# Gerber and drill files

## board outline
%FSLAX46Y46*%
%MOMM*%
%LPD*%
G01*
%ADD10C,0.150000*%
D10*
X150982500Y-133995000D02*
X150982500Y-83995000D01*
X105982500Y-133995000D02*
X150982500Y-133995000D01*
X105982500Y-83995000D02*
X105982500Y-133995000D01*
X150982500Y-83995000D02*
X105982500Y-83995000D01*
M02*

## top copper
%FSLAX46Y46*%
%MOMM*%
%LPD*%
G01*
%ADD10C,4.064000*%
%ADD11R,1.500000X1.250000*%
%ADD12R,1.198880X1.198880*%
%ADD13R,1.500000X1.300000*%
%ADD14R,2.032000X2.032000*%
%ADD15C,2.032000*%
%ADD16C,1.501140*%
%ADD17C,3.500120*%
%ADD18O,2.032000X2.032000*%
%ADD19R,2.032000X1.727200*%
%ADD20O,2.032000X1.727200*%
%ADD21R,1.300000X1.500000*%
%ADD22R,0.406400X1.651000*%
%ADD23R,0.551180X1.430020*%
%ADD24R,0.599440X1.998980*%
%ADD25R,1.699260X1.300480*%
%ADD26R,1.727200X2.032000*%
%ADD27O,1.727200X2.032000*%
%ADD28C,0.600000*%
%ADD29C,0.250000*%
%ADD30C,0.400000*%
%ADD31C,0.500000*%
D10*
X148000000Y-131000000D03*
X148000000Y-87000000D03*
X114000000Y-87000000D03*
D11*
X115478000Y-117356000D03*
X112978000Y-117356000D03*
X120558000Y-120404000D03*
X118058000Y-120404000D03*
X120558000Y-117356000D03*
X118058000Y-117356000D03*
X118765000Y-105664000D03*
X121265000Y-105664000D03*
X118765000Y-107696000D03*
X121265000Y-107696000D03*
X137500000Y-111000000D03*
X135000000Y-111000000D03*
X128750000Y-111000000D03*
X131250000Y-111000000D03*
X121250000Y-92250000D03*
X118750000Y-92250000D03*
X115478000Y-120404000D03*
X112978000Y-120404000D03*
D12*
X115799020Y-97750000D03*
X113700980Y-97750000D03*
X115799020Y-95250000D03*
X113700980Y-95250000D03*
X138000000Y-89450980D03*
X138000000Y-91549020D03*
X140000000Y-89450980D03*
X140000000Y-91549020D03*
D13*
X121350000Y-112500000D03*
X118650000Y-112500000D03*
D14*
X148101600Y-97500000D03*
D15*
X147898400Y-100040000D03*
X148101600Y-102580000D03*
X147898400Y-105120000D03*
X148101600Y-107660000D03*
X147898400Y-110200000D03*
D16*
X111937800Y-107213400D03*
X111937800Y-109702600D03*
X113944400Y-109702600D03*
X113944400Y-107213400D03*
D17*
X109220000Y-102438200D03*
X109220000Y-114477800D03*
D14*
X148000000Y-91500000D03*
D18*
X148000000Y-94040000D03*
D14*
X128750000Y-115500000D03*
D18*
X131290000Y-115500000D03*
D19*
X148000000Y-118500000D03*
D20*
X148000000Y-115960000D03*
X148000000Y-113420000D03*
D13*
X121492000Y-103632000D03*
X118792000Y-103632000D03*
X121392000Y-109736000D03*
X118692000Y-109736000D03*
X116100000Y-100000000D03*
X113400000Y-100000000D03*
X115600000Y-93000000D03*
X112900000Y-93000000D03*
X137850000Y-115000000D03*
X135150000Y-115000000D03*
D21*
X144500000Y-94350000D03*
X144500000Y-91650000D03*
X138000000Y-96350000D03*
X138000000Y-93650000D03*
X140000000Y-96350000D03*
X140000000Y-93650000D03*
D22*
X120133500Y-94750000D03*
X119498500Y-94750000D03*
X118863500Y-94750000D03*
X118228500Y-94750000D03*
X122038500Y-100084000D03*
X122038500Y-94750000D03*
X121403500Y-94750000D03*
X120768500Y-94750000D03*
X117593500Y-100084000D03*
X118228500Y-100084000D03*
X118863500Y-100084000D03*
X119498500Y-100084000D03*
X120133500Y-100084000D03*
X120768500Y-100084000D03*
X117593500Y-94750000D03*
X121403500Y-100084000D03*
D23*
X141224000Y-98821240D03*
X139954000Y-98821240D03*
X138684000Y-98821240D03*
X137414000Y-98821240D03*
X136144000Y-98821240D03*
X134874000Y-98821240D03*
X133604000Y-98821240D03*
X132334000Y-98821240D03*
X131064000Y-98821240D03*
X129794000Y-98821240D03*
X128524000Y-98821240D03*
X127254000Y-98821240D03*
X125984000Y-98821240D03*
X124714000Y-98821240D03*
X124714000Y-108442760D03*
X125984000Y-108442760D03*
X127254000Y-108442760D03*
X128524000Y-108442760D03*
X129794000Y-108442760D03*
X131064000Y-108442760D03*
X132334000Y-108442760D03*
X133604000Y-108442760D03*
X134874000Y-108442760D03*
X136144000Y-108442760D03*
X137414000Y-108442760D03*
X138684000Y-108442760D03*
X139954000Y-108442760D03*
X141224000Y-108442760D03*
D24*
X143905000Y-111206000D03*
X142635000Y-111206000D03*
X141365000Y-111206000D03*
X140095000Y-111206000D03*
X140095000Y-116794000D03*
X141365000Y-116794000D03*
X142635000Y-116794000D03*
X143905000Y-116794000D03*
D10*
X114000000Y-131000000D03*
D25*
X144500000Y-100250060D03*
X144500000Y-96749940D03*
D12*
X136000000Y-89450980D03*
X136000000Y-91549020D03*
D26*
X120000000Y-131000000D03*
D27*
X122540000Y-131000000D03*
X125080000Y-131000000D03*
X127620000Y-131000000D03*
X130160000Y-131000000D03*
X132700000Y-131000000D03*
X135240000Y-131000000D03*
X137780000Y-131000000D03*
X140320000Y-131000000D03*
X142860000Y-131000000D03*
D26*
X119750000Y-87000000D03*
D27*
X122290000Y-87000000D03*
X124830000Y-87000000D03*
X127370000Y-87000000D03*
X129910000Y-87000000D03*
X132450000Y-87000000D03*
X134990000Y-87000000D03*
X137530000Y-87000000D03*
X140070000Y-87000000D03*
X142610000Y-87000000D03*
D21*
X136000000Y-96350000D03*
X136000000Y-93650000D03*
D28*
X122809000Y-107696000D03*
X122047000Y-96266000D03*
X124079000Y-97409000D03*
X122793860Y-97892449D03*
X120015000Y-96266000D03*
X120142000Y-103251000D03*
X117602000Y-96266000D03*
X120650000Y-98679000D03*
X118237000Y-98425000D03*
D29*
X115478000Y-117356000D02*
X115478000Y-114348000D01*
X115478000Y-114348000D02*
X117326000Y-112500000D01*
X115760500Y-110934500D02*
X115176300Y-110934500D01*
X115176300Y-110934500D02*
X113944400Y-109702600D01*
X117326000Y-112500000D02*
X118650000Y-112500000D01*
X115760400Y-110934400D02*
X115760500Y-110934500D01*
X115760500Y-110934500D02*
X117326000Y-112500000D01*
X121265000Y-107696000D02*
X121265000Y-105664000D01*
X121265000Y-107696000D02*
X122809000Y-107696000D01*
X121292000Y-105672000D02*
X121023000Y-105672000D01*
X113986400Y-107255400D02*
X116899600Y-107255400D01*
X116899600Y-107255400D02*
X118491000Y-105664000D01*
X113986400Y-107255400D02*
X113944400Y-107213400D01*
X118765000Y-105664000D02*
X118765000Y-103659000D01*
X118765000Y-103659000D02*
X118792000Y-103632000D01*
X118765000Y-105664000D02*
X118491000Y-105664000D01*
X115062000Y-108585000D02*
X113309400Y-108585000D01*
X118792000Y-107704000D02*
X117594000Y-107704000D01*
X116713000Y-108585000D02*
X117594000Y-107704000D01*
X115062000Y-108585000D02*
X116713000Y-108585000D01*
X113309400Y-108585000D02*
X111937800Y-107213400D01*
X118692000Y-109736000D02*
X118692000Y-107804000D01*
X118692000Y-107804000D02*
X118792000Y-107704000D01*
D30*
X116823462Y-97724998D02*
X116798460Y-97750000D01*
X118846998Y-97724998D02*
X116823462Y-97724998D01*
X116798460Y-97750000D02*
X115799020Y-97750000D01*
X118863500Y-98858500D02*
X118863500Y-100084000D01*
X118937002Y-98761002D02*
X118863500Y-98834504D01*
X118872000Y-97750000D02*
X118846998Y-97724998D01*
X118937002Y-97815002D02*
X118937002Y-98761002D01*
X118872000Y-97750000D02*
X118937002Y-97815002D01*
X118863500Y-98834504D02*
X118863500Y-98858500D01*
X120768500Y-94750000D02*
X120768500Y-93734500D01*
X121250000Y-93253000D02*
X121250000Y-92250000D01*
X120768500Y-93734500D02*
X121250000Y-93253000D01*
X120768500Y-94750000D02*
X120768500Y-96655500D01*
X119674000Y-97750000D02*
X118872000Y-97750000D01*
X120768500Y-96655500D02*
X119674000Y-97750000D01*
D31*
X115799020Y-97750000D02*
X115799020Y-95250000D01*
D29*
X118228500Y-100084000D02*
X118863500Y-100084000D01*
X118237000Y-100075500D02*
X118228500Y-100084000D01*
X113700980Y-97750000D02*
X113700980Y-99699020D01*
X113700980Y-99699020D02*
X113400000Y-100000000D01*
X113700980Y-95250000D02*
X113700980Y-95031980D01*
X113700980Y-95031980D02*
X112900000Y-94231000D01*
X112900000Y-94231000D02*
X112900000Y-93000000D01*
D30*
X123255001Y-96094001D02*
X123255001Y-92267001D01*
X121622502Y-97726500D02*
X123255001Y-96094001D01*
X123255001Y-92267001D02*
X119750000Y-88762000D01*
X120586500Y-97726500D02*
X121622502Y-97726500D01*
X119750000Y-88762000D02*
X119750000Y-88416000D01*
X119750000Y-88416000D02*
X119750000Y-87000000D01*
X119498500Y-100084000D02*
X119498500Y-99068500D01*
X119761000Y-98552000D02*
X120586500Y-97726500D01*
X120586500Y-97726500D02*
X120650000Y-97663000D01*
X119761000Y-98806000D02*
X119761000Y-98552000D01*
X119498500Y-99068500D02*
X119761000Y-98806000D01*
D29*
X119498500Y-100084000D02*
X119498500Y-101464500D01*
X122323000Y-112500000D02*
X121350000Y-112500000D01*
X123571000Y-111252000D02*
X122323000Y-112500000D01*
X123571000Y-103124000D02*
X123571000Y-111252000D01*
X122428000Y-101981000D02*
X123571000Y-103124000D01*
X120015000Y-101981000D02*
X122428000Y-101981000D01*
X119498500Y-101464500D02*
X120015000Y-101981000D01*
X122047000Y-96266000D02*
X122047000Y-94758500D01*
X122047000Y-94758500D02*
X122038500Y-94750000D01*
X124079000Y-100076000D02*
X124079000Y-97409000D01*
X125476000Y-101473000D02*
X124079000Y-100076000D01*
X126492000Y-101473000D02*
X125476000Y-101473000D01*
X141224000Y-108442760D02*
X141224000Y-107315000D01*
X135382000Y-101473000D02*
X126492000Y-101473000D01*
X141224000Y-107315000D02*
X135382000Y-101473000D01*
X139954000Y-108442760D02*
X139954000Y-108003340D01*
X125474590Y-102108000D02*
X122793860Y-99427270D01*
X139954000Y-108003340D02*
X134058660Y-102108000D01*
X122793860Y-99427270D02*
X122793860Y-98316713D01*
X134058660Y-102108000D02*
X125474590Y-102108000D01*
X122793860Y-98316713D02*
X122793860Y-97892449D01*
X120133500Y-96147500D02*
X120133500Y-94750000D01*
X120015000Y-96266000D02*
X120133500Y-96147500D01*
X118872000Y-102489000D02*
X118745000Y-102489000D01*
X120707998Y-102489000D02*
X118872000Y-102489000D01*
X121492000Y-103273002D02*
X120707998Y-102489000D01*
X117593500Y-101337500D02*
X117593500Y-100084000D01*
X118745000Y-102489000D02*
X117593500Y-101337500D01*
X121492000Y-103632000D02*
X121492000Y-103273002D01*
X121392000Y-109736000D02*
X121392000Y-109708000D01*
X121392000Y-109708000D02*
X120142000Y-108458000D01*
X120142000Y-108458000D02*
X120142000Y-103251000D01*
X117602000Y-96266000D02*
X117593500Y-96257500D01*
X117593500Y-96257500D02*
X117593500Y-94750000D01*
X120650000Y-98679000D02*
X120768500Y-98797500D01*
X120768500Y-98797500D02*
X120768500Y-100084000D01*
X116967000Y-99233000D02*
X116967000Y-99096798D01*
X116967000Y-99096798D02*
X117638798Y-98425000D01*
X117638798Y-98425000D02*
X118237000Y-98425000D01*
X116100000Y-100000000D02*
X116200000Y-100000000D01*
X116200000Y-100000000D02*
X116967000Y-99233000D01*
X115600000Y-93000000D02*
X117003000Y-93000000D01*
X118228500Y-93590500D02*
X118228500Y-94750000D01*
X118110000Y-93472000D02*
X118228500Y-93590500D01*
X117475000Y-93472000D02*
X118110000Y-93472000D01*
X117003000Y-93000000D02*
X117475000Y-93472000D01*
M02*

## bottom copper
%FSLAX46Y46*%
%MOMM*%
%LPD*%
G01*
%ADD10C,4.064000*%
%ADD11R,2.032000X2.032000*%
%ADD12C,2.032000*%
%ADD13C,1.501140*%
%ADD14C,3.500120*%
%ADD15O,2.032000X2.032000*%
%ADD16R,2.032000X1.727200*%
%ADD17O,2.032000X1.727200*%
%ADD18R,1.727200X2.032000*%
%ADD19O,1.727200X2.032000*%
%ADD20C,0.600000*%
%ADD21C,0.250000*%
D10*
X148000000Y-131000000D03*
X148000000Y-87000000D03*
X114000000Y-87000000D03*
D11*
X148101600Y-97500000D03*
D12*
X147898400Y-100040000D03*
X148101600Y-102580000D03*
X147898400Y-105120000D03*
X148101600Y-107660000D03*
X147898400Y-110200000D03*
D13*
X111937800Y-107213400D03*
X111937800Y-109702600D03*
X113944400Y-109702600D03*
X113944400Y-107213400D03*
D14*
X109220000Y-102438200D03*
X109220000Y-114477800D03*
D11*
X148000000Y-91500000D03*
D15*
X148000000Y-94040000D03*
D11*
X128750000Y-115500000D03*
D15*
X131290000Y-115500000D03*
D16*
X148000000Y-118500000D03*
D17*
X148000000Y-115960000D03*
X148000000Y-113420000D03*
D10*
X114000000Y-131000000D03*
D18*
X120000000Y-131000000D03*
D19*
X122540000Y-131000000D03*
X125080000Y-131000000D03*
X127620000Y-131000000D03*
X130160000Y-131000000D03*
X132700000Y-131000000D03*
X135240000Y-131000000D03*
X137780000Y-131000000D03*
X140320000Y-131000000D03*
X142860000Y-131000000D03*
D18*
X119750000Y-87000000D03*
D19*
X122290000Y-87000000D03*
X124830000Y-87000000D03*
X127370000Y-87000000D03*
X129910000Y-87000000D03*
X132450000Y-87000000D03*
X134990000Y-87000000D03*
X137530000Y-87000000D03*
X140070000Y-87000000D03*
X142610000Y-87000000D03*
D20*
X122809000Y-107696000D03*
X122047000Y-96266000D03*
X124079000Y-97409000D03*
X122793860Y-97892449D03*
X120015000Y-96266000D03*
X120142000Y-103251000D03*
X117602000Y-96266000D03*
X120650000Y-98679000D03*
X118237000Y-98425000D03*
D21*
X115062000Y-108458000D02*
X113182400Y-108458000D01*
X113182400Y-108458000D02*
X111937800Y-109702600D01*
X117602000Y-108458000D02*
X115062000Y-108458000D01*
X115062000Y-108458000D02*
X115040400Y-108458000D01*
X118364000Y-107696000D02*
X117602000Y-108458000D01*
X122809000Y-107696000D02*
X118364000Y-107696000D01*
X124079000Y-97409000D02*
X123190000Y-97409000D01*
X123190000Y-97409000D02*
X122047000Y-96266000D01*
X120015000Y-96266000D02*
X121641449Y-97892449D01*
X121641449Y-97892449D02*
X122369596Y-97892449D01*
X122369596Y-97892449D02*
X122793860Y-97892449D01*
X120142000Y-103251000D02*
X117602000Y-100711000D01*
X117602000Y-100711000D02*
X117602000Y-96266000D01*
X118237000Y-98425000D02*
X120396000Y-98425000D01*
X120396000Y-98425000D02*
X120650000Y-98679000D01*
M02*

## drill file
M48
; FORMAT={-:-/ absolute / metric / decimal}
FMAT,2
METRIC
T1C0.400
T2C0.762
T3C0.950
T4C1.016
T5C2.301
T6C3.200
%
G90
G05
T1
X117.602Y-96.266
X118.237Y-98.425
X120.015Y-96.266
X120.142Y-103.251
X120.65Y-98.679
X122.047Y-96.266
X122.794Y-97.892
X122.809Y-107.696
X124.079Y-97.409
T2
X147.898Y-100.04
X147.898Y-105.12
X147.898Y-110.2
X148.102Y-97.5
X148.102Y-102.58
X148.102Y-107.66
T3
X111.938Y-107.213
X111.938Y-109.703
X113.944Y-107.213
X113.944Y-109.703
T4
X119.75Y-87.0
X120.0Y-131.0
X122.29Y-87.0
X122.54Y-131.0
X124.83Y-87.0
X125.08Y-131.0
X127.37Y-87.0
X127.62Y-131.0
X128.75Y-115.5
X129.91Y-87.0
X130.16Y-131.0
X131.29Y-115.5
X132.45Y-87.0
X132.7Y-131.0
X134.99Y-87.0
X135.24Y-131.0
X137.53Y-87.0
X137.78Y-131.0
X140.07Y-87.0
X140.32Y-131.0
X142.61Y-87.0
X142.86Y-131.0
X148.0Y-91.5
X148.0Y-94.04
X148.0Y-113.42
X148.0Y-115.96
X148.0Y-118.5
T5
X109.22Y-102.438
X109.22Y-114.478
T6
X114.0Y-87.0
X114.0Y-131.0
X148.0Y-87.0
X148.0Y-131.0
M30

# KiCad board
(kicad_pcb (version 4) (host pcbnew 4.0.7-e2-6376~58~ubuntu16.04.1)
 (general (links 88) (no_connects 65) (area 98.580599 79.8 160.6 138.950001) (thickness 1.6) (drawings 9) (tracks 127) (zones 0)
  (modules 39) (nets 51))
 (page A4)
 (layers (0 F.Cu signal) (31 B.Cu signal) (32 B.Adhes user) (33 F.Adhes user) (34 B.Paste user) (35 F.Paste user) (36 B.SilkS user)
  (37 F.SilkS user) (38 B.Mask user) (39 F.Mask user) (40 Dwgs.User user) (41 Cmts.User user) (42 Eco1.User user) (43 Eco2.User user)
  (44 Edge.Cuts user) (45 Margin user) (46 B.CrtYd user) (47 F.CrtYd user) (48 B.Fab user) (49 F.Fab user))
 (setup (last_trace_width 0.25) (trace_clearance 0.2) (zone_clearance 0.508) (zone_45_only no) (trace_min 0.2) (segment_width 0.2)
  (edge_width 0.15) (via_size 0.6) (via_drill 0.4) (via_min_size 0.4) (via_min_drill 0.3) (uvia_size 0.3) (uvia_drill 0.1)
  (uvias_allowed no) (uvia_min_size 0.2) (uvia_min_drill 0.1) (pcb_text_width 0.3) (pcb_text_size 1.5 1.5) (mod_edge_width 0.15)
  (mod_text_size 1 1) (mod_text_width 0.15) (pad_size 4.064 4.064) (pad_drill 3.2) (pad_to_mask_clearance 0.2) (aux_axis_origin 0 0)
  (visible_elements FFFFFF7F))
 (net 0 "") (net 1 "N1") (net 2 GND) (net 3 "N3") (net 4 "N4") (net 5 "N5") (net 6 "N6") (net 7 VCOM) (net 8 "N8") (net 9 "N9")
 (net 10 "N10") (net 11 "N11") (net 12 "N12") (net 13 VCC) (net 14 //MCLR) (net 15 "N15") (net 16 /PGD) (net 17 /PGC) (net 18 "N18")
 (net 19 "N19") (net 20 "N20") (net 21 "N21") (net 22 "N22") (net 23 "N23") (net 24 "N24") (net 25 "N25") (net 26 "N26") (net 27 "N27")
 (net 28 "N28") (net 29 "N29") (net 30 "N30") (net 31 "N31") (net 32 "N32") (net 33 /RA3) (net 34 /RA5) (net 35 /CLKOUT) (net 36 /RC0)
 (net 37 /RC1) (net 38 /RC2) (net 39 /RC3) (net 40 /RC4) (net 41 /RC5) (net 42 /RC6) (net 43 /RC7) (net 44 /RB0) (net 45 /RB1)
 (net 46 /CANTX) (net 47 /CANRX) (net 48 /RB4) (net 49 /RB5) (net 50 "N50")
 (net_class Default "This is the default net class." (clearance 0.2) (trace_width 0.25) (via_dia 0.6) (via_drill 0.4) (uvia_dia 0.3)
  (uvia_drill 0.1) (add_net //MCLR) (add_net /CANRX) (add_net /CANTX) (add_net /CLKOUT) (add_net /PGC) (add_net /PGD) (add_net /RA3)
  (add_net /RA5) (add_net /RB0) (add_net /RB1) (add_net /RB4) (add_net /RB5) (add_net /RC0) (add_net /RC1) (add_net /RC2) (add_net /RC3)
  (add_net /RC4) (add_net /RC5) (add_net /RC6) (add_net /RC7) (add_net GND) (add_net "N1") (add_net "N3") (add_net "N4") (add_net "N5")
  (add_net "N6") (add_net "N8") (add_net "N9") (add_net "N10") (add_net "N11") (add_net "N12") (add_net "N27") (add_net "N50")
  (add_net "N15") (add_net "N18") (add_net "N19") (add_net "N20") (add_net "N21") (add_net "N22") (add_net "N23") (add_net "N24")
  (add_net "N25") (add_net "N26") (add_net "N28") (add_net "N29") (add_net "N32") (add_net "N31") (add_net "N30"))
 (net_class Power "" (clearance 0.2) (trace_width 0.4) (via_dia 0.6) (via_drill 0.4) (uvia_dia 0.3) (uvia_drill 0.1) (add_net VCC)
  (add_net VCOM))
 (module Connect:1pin (layer F.Cu) (at 148 131 180)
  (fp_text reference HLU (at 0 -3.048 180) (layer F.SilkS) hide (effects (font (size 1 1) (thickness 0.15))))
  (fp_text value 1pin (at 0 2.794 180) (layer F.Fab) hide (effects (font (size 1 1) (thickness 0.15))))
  (pad 1 thru_hole circle (at 0 0 180) (size 4.064 4.064) (drill 3.2) (layers *.Cu *.Mask F.SilkS)))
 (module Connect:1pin (layer F.Cu) (at 148 87 180)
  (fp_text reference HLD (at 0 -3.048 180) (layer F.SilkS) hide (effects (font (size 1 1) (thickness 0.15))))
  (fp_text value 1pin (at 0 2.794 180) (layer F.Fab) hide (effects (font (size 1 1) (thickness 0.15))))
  (pad 1 thru_hole circle (at 0 0 180) (size 4.064 4.064) (drill 3.2) (layers *.Cu *.Mask F.SilkS)))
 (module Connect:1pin (layer F.Cu) (at 114 87 180)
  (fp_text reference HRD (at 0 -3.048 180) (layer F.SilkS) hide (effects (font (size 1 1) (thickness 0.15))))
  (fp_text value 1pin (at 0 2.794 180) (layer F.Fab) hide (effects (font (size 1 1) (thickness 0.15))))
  (pad 1 thru_hole circle (at 0 0 180) (size 4.064 4.064) (drill 3.2) (layers *.Cu *.Mask F.SilkS)))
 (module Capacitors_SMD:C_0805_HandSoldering (layer F.Cu) (at 114.228 117.356 180)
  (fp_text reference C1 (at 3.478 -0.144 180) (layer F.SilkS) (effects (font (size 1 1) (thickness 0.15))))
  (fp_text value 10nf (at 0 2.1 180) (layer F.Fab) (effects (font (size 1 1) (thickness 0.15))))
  (pad 1 smd rect (at -1.25 0 180) (size 1.5 1.25) (layers F.Cu F.Paste F.Mask) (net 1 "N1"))
  (pad 2 smd rect (at 1.25 0 180) (size 1.5 1.25) (layers F.Cu F.Paste F.Mask) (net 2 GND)))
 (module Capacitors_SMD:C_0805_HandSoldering (layer F.Cu) (at 119.308 120.404 180)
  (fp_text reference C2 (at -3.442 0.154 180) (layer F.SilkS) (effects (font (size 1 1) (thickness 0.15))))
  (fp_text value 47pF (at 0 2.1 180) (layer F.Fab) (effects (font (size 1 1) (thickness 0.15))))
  (pad 1 smd rect (at -1.25 0 180) (size 1.5 1.25) (layers F.Cu F.Paste F.Mask) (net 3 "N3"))
  (pad 2 smd rect (at 1.25 0 180) (size 1.5 1.25) (layers F.Cu F.Paste F.Mask) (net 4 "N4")))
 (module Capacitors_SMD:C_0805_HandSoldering (layer F.Cu) (at 119.308 117.356 180)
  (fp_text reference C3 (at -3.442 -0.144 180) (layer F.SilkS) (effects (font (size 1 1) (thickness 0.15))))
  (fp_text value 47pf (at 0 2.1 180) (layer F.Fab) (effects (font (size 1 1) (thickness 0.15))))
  (pad 1 smd rect (at -1.25 0 180) (size 1.5 1.25) (layers F.Cu F.Paste F.Mask) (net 3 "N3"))
  (pad 2 smd rect (at 1.25 0 180) (size 1.5 1.25) (layers F.Cu F.Paste F.Mask) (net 4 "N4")))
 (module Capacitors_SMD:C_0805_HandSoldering (layer F.Cu) (at 120.015 105.664)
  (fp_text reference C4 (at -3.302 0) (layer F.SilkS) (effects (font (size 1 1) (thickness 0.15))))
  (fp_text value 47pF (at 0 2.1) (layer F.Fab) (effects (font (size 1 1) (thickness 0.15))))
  (pad 1 smd rect (at -1.25 0) (size 1.5 1.25) (layers F.Cu F.Paste F.Mask) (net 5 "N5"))
  (pad 2 smd rect (at 1.25 0) (size 1.5 1.25) (layers F.Cu F.Paste F.Mask) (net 2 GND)))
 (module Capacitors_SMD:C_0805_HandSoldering (layer F.Cu) (at 120.015 107.696)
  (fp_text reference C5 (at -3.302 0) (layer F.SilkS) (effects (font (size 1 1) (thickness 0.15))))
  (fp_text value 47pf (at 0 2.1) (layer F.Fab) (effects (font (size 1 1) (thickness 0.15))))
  (pad 1 smd rect (at -1.25 0) (size 1.5 1.25) (layers F.Cu F.Paste F.Mask) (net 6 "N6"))
  (pad 2 smd rect (at 1.25 0) (size 1.5 1.25) (layers F.Cu F.Paste F.Mask) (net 2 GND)))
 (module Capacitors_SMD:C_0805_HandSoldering (layer F.Cu) (at 136.25 111 180)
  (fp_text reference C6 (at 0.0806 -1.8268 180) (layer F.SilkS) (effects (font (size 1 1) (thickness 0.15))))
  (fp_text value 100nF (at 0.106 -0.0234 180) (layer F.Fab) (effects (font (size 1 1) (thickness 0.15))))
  (pad 1 smd rect (at -1.25 0 180) (size 1.5 1.25) (layers F.Cu F.Paste F.Mask) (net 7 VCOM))
  (pad 2 smd rect (at 1.25 0 180) (size 1.5 1.25) (layers F.Cu F.Paste F.Mask) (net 2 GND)))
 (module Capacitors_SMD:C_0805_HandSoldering (layer F.Cu) (at 130 111)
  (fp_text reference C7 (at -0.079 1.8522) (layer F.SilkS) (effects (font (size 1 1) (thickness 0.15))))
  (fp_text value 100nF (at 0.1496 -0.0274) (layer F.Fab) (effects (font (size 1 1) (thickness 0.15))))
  (pad 1 smd rect (at -1.25 0) (size 1.5 1.25) (layers F.Cu F.Paste F.Mask) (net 7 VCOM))
  (pad 2 smd rect (at 1.25 0) (size 1.5 1.25) (layers F.Cu F.Paste F.Mask) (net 2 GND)))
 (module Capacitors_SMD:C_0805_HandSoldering (layer F.Cu) (at 120 92.25 180)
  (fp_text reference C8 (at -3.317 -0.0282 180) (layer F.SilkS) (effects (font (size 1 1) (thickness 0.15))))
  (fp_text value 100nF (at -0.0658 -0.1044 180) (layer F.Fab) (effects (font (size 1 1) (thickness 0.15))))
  (pad 1 smd rect (at -1.25 0 180) (size 1.5 1.25) (layers F.Cu F.Paste F.Mask) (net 7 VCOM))
  (pad 2 smd rect (at 1.25 0 180) (size 1.5 1.25) (layers F.Cu F.Paste F.Mask) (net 2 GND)))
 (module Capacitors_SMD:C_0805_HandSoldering (layer F.Cu) (at 114.228 120.404 180)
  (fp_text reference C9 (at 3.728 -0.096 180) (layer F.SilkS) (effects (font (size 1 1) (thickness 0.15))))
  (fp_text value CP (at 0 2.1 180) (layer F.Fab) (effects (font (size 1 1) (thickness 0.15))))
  (pad 1 smd rect (at -1.25 0 180) (size 1.5 1.25) (layers F.Cu F.Paste F.Mask) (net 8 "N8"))
  (pad 2 smd rect (at 1.25 0 180) (size 1.5 1.25) (layers F.Cu F.Paste F.Mask) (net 2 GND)))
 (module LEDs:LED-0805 (layer F.Cu) (at 114.75 97.75)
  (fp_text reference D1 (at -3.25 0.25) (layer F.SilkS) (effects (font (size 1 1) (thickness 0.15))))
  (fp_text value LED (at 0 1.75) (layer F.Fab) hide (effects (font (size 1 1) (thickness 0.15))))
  (pad 2 smd rect (at 1.04902 0 180) (size 1.19888 1.19888) (layers F.Cu F.Paste F.Mask) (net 7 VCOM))
  (pad 1 smd rect (at -1.04902 0 180) (size 1.19888 1.19888) (layers F.Cu F.Paste F.Mask) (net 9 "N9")))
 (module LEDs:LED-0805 (layer F.Cu) (at 114.75 95.25)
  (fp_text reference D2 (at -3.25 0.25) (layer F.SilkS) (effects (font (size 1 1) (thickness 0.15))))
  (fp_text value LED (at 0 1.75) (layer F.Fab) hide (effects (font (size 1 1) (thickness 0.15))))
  (pad 2 smd rect (at 1.04902 0 180) (size 1.19888 1.19888) (layers F.Cu F.Paste F.Mask) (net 7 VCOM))
  (pad 1 smd rect (at -1.04902 0 180) (size 1.19888 1.19888) (layers F.Cu F.Paste F.Mask) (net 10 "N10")))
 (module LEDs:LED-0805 (layer F.Cu) (at 138 90.5 90)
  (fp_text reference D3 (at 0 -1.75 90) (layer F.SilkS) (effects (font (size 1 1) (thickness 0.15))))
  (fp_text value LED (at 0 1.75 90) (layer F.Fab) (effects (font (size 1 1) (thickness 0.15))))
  (pad 2 smd rect (at 1.04902 0 270) (size 1.19888 1.19888) (layers F.Cu F.Paste F.Mask) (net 7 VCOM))
  (pad 1 smd rect (at -1.04902 0 270) (size 1.19888 1.19888) (layers F.Cu F.Paste F.Mask) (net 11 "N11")))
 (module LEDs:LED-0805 (layer F.Cu) (at 140 90.5 90)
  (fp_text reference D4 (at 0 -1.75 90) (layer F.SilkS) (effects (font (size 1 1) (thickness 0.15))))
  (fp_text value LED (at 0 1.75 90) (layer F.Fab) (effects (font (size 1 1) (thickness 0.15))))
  (pad 2 smd rect (at 1.04902 0 270) (size 1.19888 1.19888) (layers F.Cu F.Paste F.Mask) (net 7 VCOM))
  (pad 1 smd rect (at -1.04902 0 270) (size 1.19888 1.19888) (layers F.Cu F.Paste F.Mask) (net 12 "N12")))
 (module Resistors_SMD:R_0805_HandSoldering (layer F.Cu) (at 120 112.5 180)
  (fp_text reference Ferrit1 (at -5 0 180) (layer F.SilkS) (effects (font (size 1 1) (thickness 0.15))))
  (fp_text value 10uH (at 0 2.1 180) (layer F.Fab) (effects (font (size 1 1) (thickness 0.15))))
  (pad 1 smd rect (at -1.35 0 180) (size 1.5 1.3) (layers F.Cu F.Paste F.Mask) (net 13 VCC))
  (pad 2 smd rect (at 1.35 0 180) (size 1.5 1.3) (layers F.Cu F.Paste F.Mask) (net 1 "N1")))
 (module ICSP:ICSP (layer F.Cu) (at 148 97.5 270)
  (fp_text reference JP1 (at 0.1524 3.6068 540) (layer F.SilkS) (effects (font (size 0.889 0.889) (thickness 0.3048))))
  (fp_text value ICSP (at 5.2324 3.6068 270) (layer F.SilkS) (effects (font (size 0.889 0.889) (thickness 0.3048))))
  (pad 1 thru_hole rect (at 0 -0.1016 270) (size 2.032 2.032) (drill 0.762) (layers *.Cu *.Mask F.SilkS) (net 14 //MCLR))
  (pad 2 thru_hole circle (at 2.54 0.1016 270) (size 2.032 2.032) (drill 0.762) (layers *.Cu *.Mask F.SilkS) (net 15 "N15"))
  (pad 3 thru_hole circle (at 5.08 -0.1016 270) (size 2.032 2.032) (drill 0.762) (layers *.Cu *.Mask F.SilkS) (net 2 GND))
  (pad 4 thru_hole circle (at 7.62 0.1016 270) (size 2.032 2.032) (drill 0.762) (layers *.Cu *.Mask F.SilkS) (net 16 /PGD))
  (pad 5 thru_hole circle (at 10.16 -0.1016 270) (size 2.032 2.032) (drill 0.762) (layers *.Cu *.Mask F.SilkS) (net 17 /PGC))
  (pad 6 thru_hole circle (at 12.7 0.1016 270) (size 2.032 2.032) (drill 0.762) (layers *.Cu *.Mask F.SilkS) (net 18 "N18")))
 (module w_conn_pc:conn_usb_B (layer F.Cu) (at 106.934 108.458 270)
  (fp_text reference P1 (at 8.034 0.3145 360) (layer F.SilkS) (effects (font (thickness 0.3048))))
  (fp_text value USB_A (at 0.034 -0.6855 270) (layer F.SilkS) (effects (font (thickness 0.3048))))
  (pad 3 thru_hole circle (at -1.2446 -5.0038 270) (size 1.50114 1.50114) (drill 0.94996) (layers *.Cu *.Mask) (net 6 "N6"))
  (pad 4 thru_hole circle (at 1.2446 -5.0038 270) (size 1.50114 1.50114) (drill 0.94996) (layers *.Cu *.Mask) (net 2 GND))
  (pad 1 thru_hole circle (at 1.2446 -7.0104 270) (size 1.50114 1.50114) (drill 0.94996) (layers *.Cu *.Mask) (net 1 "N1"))
  (pad 2 thru_hole circle (at -1.2446 -7.0104 270) (size 1.50114 1.50114) (drill 0.94996) (layers *.Cu *.Mask) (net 5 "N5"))
  (pad "" thru_hole circle (at -6.0198 -2.286 270) (size 3.50012 3.50012) (drill 2.30124) (layers *.Cu *.Mask))
  (pad "" thru_hole circle (at 6.0198 -2.286 270) (size 3.50012 3.50012) (drill 2.30124) (layers *.Cu *.Mask)))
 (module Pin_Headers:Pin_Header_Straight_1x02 (layer F.Cu) (at 148 91.5)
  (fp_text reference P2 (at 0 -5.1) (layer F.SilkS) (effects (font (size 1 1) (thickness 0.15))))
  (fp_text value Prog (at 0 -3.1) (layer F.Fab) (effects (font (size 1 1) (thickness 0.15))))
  (pad 1 thru_hole rect (at 0 0) (size 2.032 2.032) (drill 1.016) (layers *.Cu *.Mask F.SilkS) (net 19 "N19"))
  (pad 2 thru_hole oval (at 0 2.54) (size 2.032 2.032) (drill 1.016) (layers *.Cu *.Mask F.SilkS) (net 14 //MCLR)))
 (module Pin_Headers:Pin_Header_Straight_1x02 (layer F.Cu) (at 128.75 115.5 90)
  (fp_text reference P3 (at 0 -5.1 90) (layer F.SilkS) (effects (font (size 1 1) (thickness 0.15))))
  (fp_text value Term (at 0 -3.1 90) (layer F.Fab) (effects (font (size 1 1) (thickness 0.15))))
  (pad 1 thru_hole rect (at 0 0 90) (size 2.032 2.032) (drill 1.016) (layers *.Cu *.Mask F.SilkS) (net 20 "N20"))
  (pad 2 thru_hole oval (at 0 2.54 90) (size 2.032 2.032) (drill 1.016) (layers *.Cu *.Mask F.SilkS) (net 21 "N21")))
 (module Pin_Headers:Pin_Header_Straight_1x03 (layer F.Cu) (at 148 118.5 180)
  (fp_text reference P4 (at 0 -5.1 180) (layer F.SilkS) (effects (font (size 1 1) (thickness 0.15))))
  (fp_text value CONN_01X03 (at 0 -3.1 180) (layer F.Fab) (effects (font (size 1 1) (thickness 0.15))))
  (pad 1 thru_hole rect (at 0 0 180) (size 2.032 1.7272) (drill 1.016) (layers *.Cu *.Mask F.SilkS) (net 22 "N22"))
  (pad 2 thru_hole oval (at 0 2.54 180) (size 2.032 1.7272) (drill 1.016) (layers *.Cu *.Mask F.SilkS) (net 21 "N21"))
  (pad 3 thru_hole oval (at 0 5.08 180) (size 2.032 1.7272) (drill 1.016) (layers *.Cu *.Mask F.SilkS) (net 2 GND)))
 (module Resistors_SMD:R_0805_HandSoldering (layer F.Cu) (at 120.142 103.632 180)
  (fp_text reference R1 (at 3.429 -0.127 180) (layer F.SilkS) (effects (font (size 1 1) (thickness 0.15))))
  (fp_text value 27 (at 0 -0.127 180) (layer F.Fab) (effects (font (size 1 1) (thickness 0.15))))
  (pad 1 smd rect (at -1.35 0 180) (size 1.5 1.3) (layers F.Cu F.Paste F.Mask) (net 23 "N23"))
  (pad 2 smd rect (at 1.35 0 180) (size 1.5 1.3) (layers F.Cu F.Paste F.Mask) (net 5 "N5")))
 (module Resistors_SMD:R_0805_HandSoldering (layer F.Cu) (at 120.042 109.736 180)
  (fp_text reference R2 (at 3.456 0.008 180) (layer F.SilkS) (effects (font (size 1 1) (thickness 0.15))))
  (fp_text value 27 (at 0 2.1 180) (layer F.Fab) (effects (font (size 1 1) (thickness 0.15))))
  (pad 1 smd rect (at -1.35 0 180) (size 1.5 1.3) (layers F.Cu F.Paste F.Mask) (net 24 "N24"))
  (pad 2 smd rect (at 1.35 0 180) (size 1.5 1.3) (layers F.Cu F.Paste F.Mask) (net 6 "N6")))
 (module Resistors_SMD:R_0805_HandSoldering (layer F.Cu) (at 114.75 100 180)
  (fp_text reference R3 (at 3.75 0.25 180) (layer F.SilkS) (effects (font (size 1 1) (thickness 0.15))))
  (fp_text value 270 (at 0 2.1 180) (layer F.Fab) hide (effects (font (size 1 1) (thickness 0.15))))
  (pad 1 smd rect (at -1.35 0 180) (size 1.5 1.3) (layers F.Cu F.Paste F.Mask) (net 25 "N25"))
  (pad 2 smd rect (at 1.35 0 180) (size 1.5 1.3) (layers F.Cu F.Paste F.Mask) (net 9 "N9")))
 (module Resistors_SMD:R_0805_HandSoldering (layer F.Cu) (at 114.25 93 180)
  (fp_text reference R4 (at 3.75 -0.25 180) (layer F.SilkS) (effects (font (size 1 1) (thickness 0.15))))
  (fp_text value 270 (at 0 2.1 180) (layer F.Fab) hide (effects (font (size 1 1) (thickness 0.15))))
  (pad 1 smd rect (at -1.35 0 180) (size 1.5 1.3) (layers F.Cu F.Paste F.Mask) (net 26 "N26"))
  (pad 2 smd rect (at 1.35 0 180) (size 1.5 1.3) (layers F.Cu F.Paste F.Mask) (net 10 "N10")))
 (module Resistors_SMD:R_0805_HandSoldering (layer F.Cu) (at 136.5 115 180)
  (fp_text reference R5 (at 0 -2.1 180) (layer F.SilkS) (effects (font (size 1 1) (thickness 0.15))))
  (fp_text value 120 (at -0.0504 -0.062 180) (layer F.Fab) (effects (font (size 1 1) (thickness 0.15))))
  (pad 1 smd rect (at -1.35 0 180) (size 1.5 1.3) (layers F.Cu F.Paste F.Mask) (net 22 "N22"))
  (pad 2 smd rect (at 1.35 0 180) (size 1.5 1.3) (layers F.Cu F.Paste F.Mask) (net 20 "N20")))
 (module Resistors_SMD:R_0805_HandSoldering (layer F.Cu) (at 144.5 93 90)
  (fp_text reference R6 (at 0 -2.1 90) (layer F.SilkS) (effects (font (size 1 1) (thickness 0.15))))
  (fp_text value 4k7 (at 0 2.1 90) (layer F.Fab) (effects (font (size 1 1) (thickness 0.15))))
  (pad 1 smd rect (at -1.35 0 90) (size 1.5 1.3) (layers F.Cu F.Paste F.Mask) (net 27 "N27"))
  (pad 2 smd rect (at 1.35 0 90) (size 1.5 1.3) (layers F.Cu F.Paste F.Mask) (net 7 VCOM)))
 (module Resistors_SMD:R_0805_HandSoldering (layer F.Cu) (at 138 95 90)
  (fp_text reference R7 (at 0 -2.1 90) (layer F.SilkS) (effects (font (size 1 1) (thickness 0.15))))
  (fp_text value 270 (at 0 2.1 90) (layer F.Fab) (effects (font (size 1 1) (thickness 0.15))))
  (pad 1 smd rect (at -1.35 0 90) (size 1.5 1.3) (layers F.Cu F.Paste F.Mask) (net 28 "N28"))
  (pad 2 smd rect (at 1.35 0 90) (size 1.5 1.3) (layers F.Cu F.Paste F.Mask) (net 11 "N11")))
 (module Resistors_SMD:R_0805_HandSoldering (layer F.Cu) (at 140 95 90)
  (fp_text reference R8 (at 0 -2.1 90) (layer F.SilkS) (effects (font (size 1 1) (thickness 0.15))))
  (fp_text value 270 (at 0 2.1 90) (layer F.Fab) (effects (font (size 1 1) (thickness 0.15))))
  (pad 1 smd rect (at -1.35 0 90) (size 1.5 1.3) (layers F.Cu F.Paste F.Mask) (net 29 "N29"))
  (pad 2 smd rect (at 1.35 0 90) (size 1.5 1.3) (layers F.Cu F.Paste F.Mask) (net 12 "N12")))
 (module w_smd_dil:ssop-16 (layer F.Cu) (at 119.816 97.417 180)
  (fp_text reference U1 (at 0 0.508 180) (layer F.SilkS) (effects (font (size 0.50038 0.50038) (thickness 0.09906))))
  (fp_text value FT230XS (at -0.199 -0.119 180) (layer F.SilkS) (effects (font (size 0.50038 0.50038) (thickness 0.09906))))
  (pad 4 smd rect (at -0.3175 2.667 180) (size 0.4064 1.651) (layers F.Cu F.Paste F.Mask) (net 17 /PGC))
  (pad 5 smd rect (at 0.3175 2.667 180) (size 0.4064 1.651) (layers F.Cu F.Paste F.Mask) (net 2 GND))
  (pad 6 smd rect (at 0.9525 2.667 180) (size 0.4064 1.651) (layers F.Cu F.Paste F.Mask) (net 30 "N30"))
  (pad 7 smd rect (at 1.5875 2.667 180) (size 0.4064 1.651) (layers F.Cu F.Paste F.Mask) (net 26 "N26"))
  (pad 16 smd rect (at -2.2225 -2.667 180) (size 0.4064 1.651) (layers F.Cu F.Paste F.Mask) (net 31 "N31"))
  (pad 1 smd rect (at -2.2225 2.667 180) (size 0.4064 1.651) (layers F.Cu F.Paste F.Mask) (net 16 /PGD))
  (pad 2 smd rect (at -1.5875 2.667 180) (size 0.4064 1.651) (layers F.Cu F.Paste F.Mask) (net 19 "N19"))
  (pad 3 smd rect (at -0.9525 2.667 180) (size 0.4064 1.651) (layers F.Cu F.Paste F.Mask) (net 7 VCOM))
  (pad 9 smd rect (at 2.2225 -2.667 180) (size 0.4064 1.651) (layers F.Cu F.Paste F.Mask) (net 23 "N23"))
  (pad 10 smd rect (at 1.5875 -2.667 180) (size 0.4064 1.651) (layers F.Cu F.Paste F.Mask) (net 7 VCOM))
  (pad 11 smd rect (at 0.9525 -2.667 180) (size 0.4064 1.651) (layers F.Cu F.Paste F.Mask) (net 7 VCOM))
  (pad 12 smd rect (at 0.3175 -2.667 180) (size 0.4064 1.651) (layers F.Cu F.Paste F.Mask) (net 13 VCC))
  (pad 13 smd rect (at -0.3175 -2.667 180) (size 0.4064 1.651) (layers F.Cu F.Paste F.Mask) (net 2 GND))
  (pad 14 smd rect (at -0.9525 -2.667 180) (size 0.4064 1.651) (layers F.Cu F.Paste F.Mask) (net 25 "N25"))
  (pad 8 smd rect (at 2.2225 2.667 180) (size 0.4064 1.651) (layers F.Cu F.Paste F.Mask) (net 24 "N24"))
  (pad 15 smd rect (at -1.5875 -2.667 180) (size 0.4064 1.651) (layers F.Cu F.Paste F.Mask) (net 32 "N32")))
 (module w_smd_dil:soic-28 (layer F.Cu) (at 132.969 103.632 180)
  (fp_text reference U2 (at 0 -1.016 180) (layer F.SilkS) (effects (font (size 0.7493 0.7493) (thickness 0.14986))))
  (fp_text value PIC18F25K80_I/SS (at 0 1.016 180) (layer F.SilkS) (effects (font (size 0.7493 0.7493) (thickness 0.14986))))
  (pad 1 smd rect (at -8.255 4.81076 180) (size 0.55118 1.43002) (layers F.Cu F.Paste F.Mask) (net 14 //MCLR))
  (pad 2 smd rect (at -6.985 4.81076 180) (size 0.55118 1.43002) (layers F.Cu F.Paste F.Mask) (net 30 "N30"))
  (pad 3 smd rect (at -5.715 4.81076 180) (size 0.55118 1.43002) (layers F.Cu F.Paste F.Mask) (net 29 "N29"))
  (pad 4 smd rect (at -4.445 4.81076 180) (size 0.55118 1.43002) (layers F.Cu F.Paste F.Mask) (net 28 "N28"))
  (pad 5 smd rect (at -3.175 4.81076 180) (size 0.55118 1.43002) (layers F.Cu F.Paste F.Mask) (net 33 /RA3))
  (pad 6 smd rect (at -1.905 4.81076 180) (size 0.55118 1.43002) (layers F.Cu F.Paste F.Mask) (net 8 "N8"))
  (pad 7 smd rect (at -0.635 4.81076 180) (size 0.55118 1.43002) (layers F.Cu F.Paste F.Mask) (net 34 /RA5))
  (pad 8 smd rect (at 0.635 4.81076 180) (size 0.55118 1.43002) (layers F.Cu F.Paste F.Mask) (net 2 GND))
  (pad 9 smd rect (at 1.905 4.81076 180) (size 0.55118 1.43002) (layers F.Cu F.Paste F.Mask) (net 31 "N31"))
  (pad 10 smd rect (at 3.175 4.81076 180) (size 0.55118 1.43002) (layers F.Cu F.Paste F.Mask) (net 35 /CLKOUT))
  (pad 11 smd rect (at 4.445 4.81076 180) (size 0.55118 1.43002) (layers F.Cu F.Paste F.Mask) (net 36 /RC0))
  (pad 12 smd rect (at 5.715 4.81076 180) (size 0.55118 1.43002) (layers F.Cu F.Paste F.Mask) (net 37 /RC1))
  (pad 13 smd rect (at 6.985 4.81076 180) (size 0.55118 1.43002) (layers F.Cu F.Paste F.Mask) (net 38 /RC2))
  (pad 14 smd rect (at 8.255 4.81076 180) (size 0.55118 1.43002) (layers F.Cu F.Paste F.Mask) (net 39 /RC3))
  (pad 15 smd rect (at 8.255 -4.81076 180) (size 0.55118 1.43002) (layers F.Cu F.Paste F.Mask) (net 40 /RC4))
  (pad 16 smd rect (at 6.985 -4.81076 180) (size 0.55118 1.43002) (layers F.Cu F.Paste F.Mask) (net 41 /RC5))
  (pad 17 smd rect (at 5.715 -4.81076 180) (size 0.55118 1.43002) (layers F.Cu F.Paste F.Mask) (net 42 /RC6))
  (pad 18 smd rect (at 4.445 -4.81076 180) (size 0.55118 1.43002) (layers F.Cu F.Paste F.Mask) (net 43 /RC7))
  (pad 19 smd rect (at 3.175 -4.81076 180) (size 0.55118 1.43002) (layers F.Cu F.Paste F.Mask) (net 2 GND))
  (pad 20 smd rect (at 1.905 -4.81076 180) (size 0.55118 1.43002) (layers F.Cu F.Paste F.Mask))
  (pad 21 smd rect (at 0.635 -4.81076 180) (size 0.55118 1.43002) (layers F.Cu F.Paste F.Mask) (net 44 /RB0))
  (pad 22 smd rect (at -0.635 -4.81076 180) (size 0.55118 1.43002) (layers F.Cu F.Paste F.Mask) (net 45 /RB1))
  (pad 23 smd rect (at -1.905 -4.81076 180) (size 0.55118 1.43002) (layers F.Cu F.Paste F.Mask) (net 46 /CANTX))
  (pad 24 smd rect (at -3.175 -4.81076 180) (size 0.55118 1.43002) (layers F.Cu F.Paste F.Mask) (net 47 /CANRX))
  (pad 25 smd rect (at -4.445 -4.81076 180) (size 0.55118 1.43002) (layers F.Cu F.Paste F.Mask) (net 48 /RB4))
  (pad 26 smd rect (at -5.715 -4.81076 180) (size 0.55118 1.43002) (layers F.Cu F.Paste F.Mask) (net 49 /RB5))
  (pad 27 smd rect (at -6.985 -4.81076 180) (size 0.55118 1.43002) (layers F.Cu F.Paste F.Mask) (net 17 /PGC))
  (pad 28 smd rect (at -8.255 -4.81076 180) (size 0.55118 1.43002) (layers F.Cu F.Paste F.Mask) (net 16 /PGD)))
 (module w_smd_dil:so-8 (layer F.Cu) (at 142 114 180)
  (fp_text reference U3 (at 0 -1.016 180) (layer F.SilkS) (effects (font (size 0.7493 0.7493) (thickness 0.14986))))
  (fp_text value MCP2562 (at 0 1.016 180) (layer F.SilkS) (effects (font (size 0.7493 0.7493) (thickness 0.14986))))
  (pad 1 smd rect (at -1.905 2.794 180) (size 0.59944 1.99898) (layers F.Cu F.Paste F.Mask) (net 46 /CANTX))
  (pad 2 smd rect (at -0.635 2.794 180) (size 0.59944 1.99898) (layers F.Cu F.Paste F.Mask) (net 2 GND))
  (pad 3 smd rect (at 0.635 2.794 180) (size 0.59944 1.99898) (layers F.Cu F.Paste F.Mask) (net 13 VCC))
  (pad 4 smd rect (at 1.905 2.794 180) (size 0.59944 1.99898) (layers F.Cu F.Paste F.Mask) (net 47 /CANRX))
  (pad 5 smd rect (at 1.905 -2.794 180) (size 0.59944 1.99898) (layers F.Cu F.Paste F.Mask) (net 7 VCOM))
  (pad 6 smd rect (at 0.635 -2.794 180) (size 0.59944 1.99898) (layers F.Cu F.Paste F.Mask) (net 21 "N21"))
  (pad 7 smd rect (at -0.635 -2.794 180) (size 0.59944 1.99898) (layers F.Cu F.Paste F.Mask) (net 22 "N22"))
  (pad 8 smd rect (at -1.905 -2.794 180) (size 0.59944 1.99898) (layers F.Cu F.Paste F.Mask) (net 2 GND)))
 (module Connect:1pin (layer F.Cu) (at 114 131 180)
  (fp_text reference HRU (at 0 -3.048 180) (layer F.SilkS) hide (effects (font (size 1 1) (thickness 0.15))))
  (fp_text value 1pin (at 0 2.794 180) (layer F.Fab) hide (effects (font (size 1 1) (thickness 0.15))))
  (pad 1 thru_hole circle (at 0 0 180) (size 4.064 4.064) (drill 3.2) (layers *.Cu *.Mask F.SilkS)))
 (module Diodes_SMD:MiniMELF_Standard (layer F.Cu) (at 144.5 98.5 90)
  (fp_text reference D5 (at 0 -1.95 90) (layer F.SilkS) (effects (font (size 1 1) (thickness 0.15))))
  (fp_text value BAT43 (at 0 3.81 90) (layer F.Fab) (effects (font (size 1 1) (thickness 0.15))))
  (pad 1 smd rect (at -1.75006 0 90) (size 1.30048 1.69926) (layers F.Cu F.Paste F.Mask) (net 14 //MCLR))
  (pad 2 smd rect (at 1.75006 0 90) (size 1.30048 1.69926) (layers F.Cu F.Paste F.Mask) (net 27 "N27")))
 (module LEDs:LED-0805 (layer F.Cu) (at 136 90.5 90)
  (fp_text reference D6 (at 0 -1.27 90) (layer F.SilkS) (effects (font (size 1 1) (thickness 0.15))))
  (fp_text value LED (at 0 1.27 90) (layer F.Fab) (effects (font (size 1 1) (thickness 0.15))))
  (pad 2 smd rect (at 1.04902 0 270) (size 1.19888 1.19888) (layers F.Cu F.Paste F.Mask) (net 7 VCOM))
  (pad 1 smd rect (at -1.04902 0 270) (size 1.19888 1.19888) (layers F.Cu F.Paste F.Mask) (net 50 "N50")))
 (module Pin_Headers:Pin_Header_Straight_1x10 (layer F.Cu) (at 120 131 90)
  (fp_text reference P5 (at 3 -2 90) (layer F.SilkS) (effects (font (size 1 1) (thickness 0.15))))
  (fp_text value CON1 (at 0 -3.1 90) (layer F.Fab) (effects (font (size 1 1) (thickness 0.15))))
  (pad 1 thru_hole rect (at 0 0 90) (size 2.032 1.7272) (drill 1.016) (layers *.Cu *.Mask F.SilkS) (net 7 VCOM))
  (pad 2 thru_hole oval (at 0 2.54 90) (size 2.032 1.7272) (drill 1.016) (layers *.Cu *.Mask F.SilkS) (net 2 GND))
  (pad 3 thru_hole oval (at 0 5.08 90) (size 2.032 1.7272) (drill 1.016) (layers *.Cu *.Mask F.SilkS) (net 44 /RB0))
  (pad 4 thru_hole oval (at 0 7.62 90) (size 2.032 1.7272) (drill 1.016) (layers *.Cu *.Mask F.SilkS) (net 45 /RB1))
  (pad 5 thru_hole oval (at 0 10.16 90) (size 2.032 1.7272) (drill 1.016) (layers *.Cu *.Mask F.SilkS) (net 46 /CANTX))
  (pad 6 thru_hole oval (at 0 12.7 90) (size 2.032 1.7272) (drill 1.016) (layers *.Cu *.Mask F.SilkS) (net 47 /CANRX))
  (pad 7 thru_hole oval (at 0 15.24 90) (size 2.032 1.7272) (drill 1.016) (layers *.Cu *.Mask F.SilkS) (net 48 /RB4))
  (pad 8 thru_hole oval (at 0 17.78 90) (size 2.032 1.7272) (drill 1.016) (layers *.Cu *.Mask F.SilkS) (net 49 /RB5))
  (pad 9 thru_hole oval (at 0 20.32 90) (size 2.032 1.7272) (drill 1.016) (layers *.Cu *.Mask F.SilkS) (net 34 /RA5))
  (pad 10 thru_hole oval (at 0 22.86 90) (size 2.032 1.7272) (drill 1.016) (layers *.Cu *.Mask F.SilkS) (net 35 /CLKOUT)))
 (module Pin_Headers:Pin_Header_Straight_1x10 (layer F.Cu) (at 119.75 87 90)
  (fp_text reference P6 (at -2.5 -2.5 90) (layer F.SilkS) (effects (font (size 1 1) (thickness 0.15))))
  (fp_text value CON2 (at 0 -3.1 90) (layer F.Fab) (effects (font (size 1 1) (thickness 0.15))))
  (pad 1 thru_hole rect (at 0 0 90) (size 2.032 1.7272) (drill 1.016) (layers *.Cu *.Mask F.SilkS) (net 13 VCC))
  (pad 2 thru_hole oval (at 0 2.54 90) (size 2.032 1.7272) (drill 1.016) (layers *.Cu *.Mask F.SilkS) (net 2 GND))
  (pad 3 thru_hole oval (at 0 5.08 90) (size 2.032 1.7272) (drill 1.016) (layers *.Cu *.Mask F.SilkS) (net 36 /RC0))
  (pad 4 thru_hole oval (at 0 7.62 90) (size 2.032 1.7272) (drill 1.016) (layers *.Cu *.Mask F.SilkS) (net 37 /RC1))
  (pad 5 thru_hole oval (at 0 10.16 90) (size 2.032 1.7272) (drill 1.016) (layers *.Cu *.Mask F.SilkS) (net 38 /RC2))
  (pad 6 thru_hole oval (at 0 12.7 90) (size 2.032 1.7272) (drill 1.016) (layers *.Cu *.Mask F.SilkS) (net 39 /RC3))
  (pad 7 thru_hole oval (at 0 15.24 90) (size 2.032 1.7272) (drill 1.016) (layers *.Cu *.Mask F.SilkS) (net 40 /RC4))
  (pad 8 thru_hole oval (at 0 17.78 90) (size 2.032 1.7272) (drill 1.016) (layers *.Cu *.Mask F.SilkS) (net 41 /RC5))
  (pad 9 thru_hole oval (at 0 20.32 90) (size 2.032 1.7272) (drill 1.016) (layers *.Cu *.Mask F.SilkS) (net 42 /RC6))
  (pad 10 thru_hole oval (at 0 22.86 90) (size 2.032 1.7272) (drill 1.016) (layers *.Cu *.Mask F.SilkS) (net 43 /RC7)))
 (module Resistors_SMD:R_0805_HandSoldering (layer F.Cu) (at 136 95 90)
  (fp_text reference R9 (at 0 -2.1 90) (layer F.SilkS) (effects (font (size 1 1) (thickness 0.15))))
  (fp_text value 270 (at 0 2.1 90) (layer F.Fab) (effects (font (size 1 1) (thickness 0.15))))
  (pad 1 smd rect (at -1.35 0 90) (size 1.5 1.3) (layers F.Cu F.Paste F.Mask) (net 33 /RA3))
  (pad 2 smd rect (at 1.35 0 90) (size 1.5 1.3) (layers F.Cu F.Paste F.Mask) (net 50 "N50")))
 (gr_line (start 150.9825 133.995) (end 150.9825 83.995) (angle 90) (layer Edge.Cuts) (width 0.15))
 (gr_line (start 105.9825 133.995) (end 150.9825 133.995) (angle 90) (layer Edge.Cuts) (width 0.15))
 (gr_line (start 105.9825 83.995) (end 105.9825 133.995) (angle 90) (layer Edge.Cuts) (width 0.15))
 (gr_line (start 150.9825 83.995) (end 105.9825 83.995) (angle 90) (layer Edge.Cuts) (width 0.15))
 (segment (start 115.478 117.356) (end 115.478 114.348) (width 0.25) (layer F.Cu) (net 1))
 (segment (start 115.478 114.348) (end 117.326 112.5) (width 0.25) (layer F.Cu) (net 1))
 (segment (start 115.7605 110.9345) (end 115.1763 110.9345) (width 0.25) (layer F.Cu) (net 1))
 (segment (start 115.1763 110.9345) (end 113.9444 109.7026) (width 0.25) (layer F.Cu) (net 1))
 (segment (start 117.326 112.5) (end 118.65 112.5) (width 0.25) (layer F.Cu) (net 1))
 (segment (start 115.7604 110.9344) (end 115.7605 110.9345) (width 0.25) (layer F.Cu) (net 1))
 (segment (start 115.7605 110.9345) (end 117.326 112.5) (width 0.25) (layer F.Cu) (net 1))
 (segment (start 115.062 108.458) (end 113.1824 108.458) (width 0.25) (layer B.Cu) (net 2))
 (segment (start 113.1824 108.458) (end 111.9378 109.7026) (width 0.25) (layer B.Cu) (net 2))
 (segment (start 117.602 108.458) (end 115.062 108.458) (width 0.25) (layer B.Cu) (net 2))
 (segment (start 115.062 108.458) (end 115.0404 108.458) (width 0.25) (layer B.Cu) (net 2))
 (segment (start 118.364 107.696) (end 117.602 108.458) (width 0.25) (layer B.Cu) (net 2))
 (segment (start 122.809 107.696) (end 118.364 107.696) (width 0.25) (layer B.Cu) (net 2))
 (segment (start 121.265 107.696) (end 121.265 105.664) (width 0.25) (layer F.Cu) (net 2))
 (segment (start 121.265 107.696) (end 122.809 107.696) (width 0.25) (layer F.Cu) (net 2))
 (via (at 122.809 107.696) (size 0.6) (drill 0.4) (layers F.Cu B.Cu) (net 2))
 (segment (start 121.292 105.672) (end 121.023 105.672) (width 0.25) (layer F.Cu) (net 2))
 (segment (start 113.9864 107.2554) (end 116.8996 107.2554) (width 0.25) (layer F.Cu) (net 5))
 (segment (start 116.8996 107.2554) (end 118.491 105.664) (width 0.25) (layer F.Cu) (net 5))
 (segment (start 113.9864 107.2554) (end 113.9444 107.2134) (width 0.25) (layer F.Cu) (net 5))
 (segment (start 118.765 105.664) (end 118.765 103.659) (width 0.25) (layer F.Cu) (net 5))
 (segment (start 118.765 103.659) (end 118.792 103.632) (width 0.25) (layer F.Cu) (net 5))
 (segment (start 118.765 105.664) (end 118.491 105.664) (width 0.25) (layer F.Cu) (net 5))
 (segment (start 115.062 108.585) (end 113.3094 108.585) (width 0.25) (layer F.Cu) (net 6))
 (segment (start 118.792 107.704) (end 117.594 107.704) (width 0.25) (layer F.Cu) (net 6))
 (segment (start 116.713 108.585) (end 117.594 107.704) (width 0.25) (layer F.Cu) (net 6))
 (segment (start 115.062 108.585) (end 116.713 108.585) (width 0.25) (layer F.Cu) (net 6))
 (segment (start 113.3094 108.585) (end 111.9378 107.2134) (width 0.25) (layer F.Cu) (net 6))
 (segment (start 118.692 109.736) (end 118.692 107.804) (width 0.25) (layer F.Cu) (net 6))
 (segment (start 118.692 107.804) (end 118.792 107.704) (width 0.25) (layer F.Cu) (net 6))
 (segment (start 116.823462 97.724998) (end 116.79846 97.75) (width 0.4) (layer F.Cu) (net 7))
 (segment (start 118.846998 97.724998) (end 116.823462 97.724998) (width 0.4) (layer F.Cu) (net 7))
 (segment (start 116.79846 97.75) (end 115.79902 97.75) (width 0.4) (layer F.Cu) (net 7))
 (segment (start 118.8635 98.8585) (end 118.8635 100.084) (width 0.4) (layer F.Cu) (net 7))
 (segment (start 118.937002 98.761002) (end 118.8635 98.834504) (width 0.4) (layer F.Cu) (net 7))
 (segment (start 118.872 97.75) (end 118.846998 97.724998) (width 0.4) (layer F.Cu) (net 7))
 (segment (start 118.937002 97.815002) (end 118.937002 98.761002) (width 0.4) (layer F.Cu) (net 7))
 (segment (start 118.872 97.75) (end 118.937002 97.815002) (width 0.4) (layer F.Cu) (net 7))
 (segment (start 118.8635 98.834504) (end 118.8635 98.8585) (width 0.4) (layer F.Cu) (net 7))
 (segment (start 120.7685 94.75) (end 120.7685 93.7345) (width 0.4) (layer F.Cu) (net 7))
 (segment (start 121.25 93.253) (end 121.25 92.25) (width 0.4) (layer F.Cu) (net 7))
 (segment (start 120.7685 93.7345) (end 121.25 93.253) (width 0.4) (layer F.Cu) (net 7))
 (segment (start 120.7685 94.75) (end 120.7685 96.6555) (width 0.4) (layer F.Cu) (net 7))
 (segment (start 119.674 97.75) (end 118.872 97.75) (width 0.4) (layer F.Cu) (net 7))
 (segment (start 120.7685 96.6555) (end 119.674 97.75) (width 0.4) (layer F.Cu) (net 7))
 (segment (start 115.79902 97.75) (end 115.79902 95.25) (width 0.5) (layer F.Cu) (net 7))
 (segment (start 118.2285 100.084) (end 118.8635 100.084) (width 0.25) (layer F.Cu) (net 7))
 (segment (start 118.237 100.0755) (end 118.2285 100.084) (width 0.25) (layer F.Cu) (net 7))
 (segment (start 113.70098 97.75) (end 113.70098 99.69902) (width 0.25) (layer F.Cu) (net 9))
 (segment (start 113.70098 99.69902) (end 113.4 100) (width 0.25) (layer F.Cu) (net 9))
 (segment (start 113.70098 95.25) (end 113.70098 95.03198) (width 0.25) (layer F.Cu) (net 10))
 (segment (start 113.70098 95.03198) (end 112.9 94.231) (width 0.25) (layer F.Cu) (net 10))
 (segment (start 112.9 94.231) (end 112.9 93) (width 0.25) (layer F.Cu) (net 10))
 (segment (start 123.255001 96.094001) (end 123.255001 92.267001) (width 0.4) (layer F.Cu) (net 13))
 (segment (start 121.622502 97.7265) (end 123.255001 96.094001) (width 0.4) (layer F.Cu) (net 13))
 (segment (start 123.255001 92.267001) (end 119.75 88.762) (width 0.4) (layer F.Cu) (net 13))
 (segment (start 120.5865 97.7265) (end 121.622502 97.7265) (width 0.4) (layer F.Cu) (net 13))
 (segment (start 119.75 88.762) (end 119.75 88.416) (width 0.4) (layer F.Cu) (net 13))
 (segment (start 119.75 88.416) (end 119.75 87) (width 0.4) (layer F.Cu) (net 13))
 (segment (start 119.4985 100.084) (end 119.4985 99.0685) (width 0.4) (layer F.Cu) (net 13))
 (segment (start 119.761 98.552) (end 120.5865 97.7265) (width 0.4) (layer F.Cu) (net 13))
 (segment (start 120.5865 97.7265) (end 120.65 97.663) (width 0.4) (layer F.Cu) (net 13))
 (segment (start 119.761 98.806) (end 119.761 98.552) (width 0.4) (layer F.Cu) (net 13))
 (segment (start 119.4985 99.0685) (end 119.761 98.806) (width 0.4) (layer F.Cu) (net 13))
 (segment (start 119.4985 100.084) (end 119.4985 101.4645) (width 0.25) (layer F.Cu) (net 13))
 (segment (start 122.323 112.5) (end 121.35 112.5) (width 0.25) (layer F.Cu) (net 13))
 (segment (start 123.571 111.252) (end 122.323 112.5) (width 0.25) (layer F.Cu) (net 13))
 (segment (start 123.571 103.124) (end 123.571 111.252) (width 0.25) (layer F.Cu) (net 13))
 (segment (start 122.428 101.981) (end 123.571 103.124) (width 0.25) (layer F.Cu) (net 13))
 (segment (start 120.015 101.981) (end 122.428 101.981) (width 0.25) (layer F.Cu) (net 13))
 (segment (start 119.4985 101.4645) (end 120.015 101.981) (width 0.25) (layer F.Cu) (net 13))
 (segment (start 122.047 96.266) (end 122.047 94.7585) (width 0.25) (layer F.Cu) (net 16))
 (segment (start 122.047 94.7585) (end 122.0385 94.75) (width 0.25) (layer F.Cu) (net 16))
 (segment (start 124.079 97.409) (end 123.19 97.409) (width 0.25) (layer B.Cu) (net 16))
 (segment (start 123.19 97.409) (end 122.047 96.266) (width 0.25) (layer B.Cu) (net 16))
 (via (at 122.047 96.266) (size 0.6) (drill 0.4) (layers F.Cu B.Cu) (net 16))
 (segment (start 124.079 100.076) (end 124.079 97.409) (width 0.25) (layer F.Cu) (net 16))
 (segment (start 125.476 101.473) (end 124.079 100.076) (width 0.25) (layer F.Cu) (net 16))
 (via (at 124.079 97.409) (size 0.6) (drill 0.4) (layers F.Cu B.Cu) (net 16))
 (segment (start 126.492 101.473) (end 125.476 101.473) (width 0.25) (layer F.Cu) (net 16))
 (segment (start 141.224 108.44276) (end 141.224 107.315) (width 0.25) (layer F.Cu) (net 16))
 (segment (start 135.382 101.473) (end 126.492 101.473) (width 0.25) (layer F.Cu) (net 16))
 (segment (start 141.224 107.315) (end 135.382 101.473) (width 0.25) (layer F.Cu) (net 16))
 (segment (start 139.954 108.44276) (end 139.954 108.00334) (width 0.25) (layer F.Cu) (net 17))
 (segment (start 120.015 96.266) (end 121.641449 97.892449) (width 0.25) (layer B.Cu) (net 17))
 (segment (start 121.641449 97.892449) (end 122.369596 97.892449) (width 0.25) (layer B.Cu) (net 17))
 (segment (start 125.47459 102.108) (end 122.79386 99.42727) (width 0.25) (layer F.Cu) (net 17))
 (segment (start 139.954 108.00334) (end 134.05866 102.108) (width 0.25) (layer F.Cu) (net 17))
 (segment (start 122.79386 99.42727) (end 122.79386 98.316713) (width 0.25) (layer F.Cu) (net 17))
 (segment (start 134.05866 102.108) (end 125.47459 102.108) (width 0.25) (layer F.Cu) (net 17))
 (via (at 122.79386 97.892449) (size 0.6) (drill 0.4) (layers F.Cu B.Cu) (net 17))
 (segment (start 122.79386 98.316713) (end 122.79386 97.892449) (width 0.25) (layer F.Cu) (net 17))
 (segment (start 122.369596 97.892449) (end 122.79386 97.892449) (width 0.25) (layer B.Cu) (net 17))
 (segment (start 120.1335 96.1475) (end 120.1335 94.75) (width 0.25) (layer F.Cu) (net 17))
 (segment (start 120.015 96.266) (end 120.1335 96.1475) (width 0.25) (layer F.Cu) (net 17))
 (via (at 120.015 96.266) (size 0.6) (drill 0.4) (layers F.Cu B.Cu) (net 17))
 (segment (start 118.872 102.489) (end 118.745 102.489) (width 0.25) (layer F.Cu) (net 23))
 (segment (start 120.707998 102.489) (end 118.872 102.489) (width 0.25) (layer F.Cu) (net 23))
 (segment (start 121.492 103.273002) (end 120.707998 102.489) (width 0.25) (layer F.Cu) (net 23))
 (segment (start 117.5935 101.3375) (end 117.5935 100.084) (width 0.25) (layer F.Cu) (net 23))
 (segment (start 118.745 102.489) (end 117.5935 101.3375) (width 0.25) (layer F.Cu) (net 23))
 (segment (start 121.492 103.632) (end 121.492 103.273002) (width 0.25) (layer F.Cu) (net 23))
 (segment (start 121.392 109.736) (end 121.392 109.708) (width 0.25) (layer F.Cu) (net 24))
 (segment (start 121.392 109.708) (end 120.142 108.458) (width 0.25) (layer F.Cu) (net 24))
 (segment (start 120.142 108.458) (end 120.142 103.251) (width 0.25) (layer F.Cu) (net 24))
 (via (at 120.142 103.251) (size 0.6) (drill 0.4) (layers F.Cu B.Cu) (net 24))
 (segment (start 120.142 103.251) (end 117.602 100.711) (width 0.25) (layer B.Cu) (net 24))
 (segment (start 117.602 100.711) (end 117.602 96.266) (width 0.25) (layer B.Cu) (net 24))
 (via (at 117.602 96.266) (size 0.6) (drill 0.4) (layers F.Cu B.Cu) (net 24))
 (segment (start 117.602 96.266) (end 117.5935 96.2575) (width 0.25) (layer F.Cu) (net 24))
 (segment (start 117.5935 96.2575) (end 117.5935 94.75) (width 0.25) (layer F.Cu) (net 24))
 (segment (start 120.65 98.679) (end 120.7685 98.7975) (width 0.25) (layer F.Cu) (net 25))
 (segment (start 120.7685 98.7975) (end 120.7685 100.084) (width 0.25) (layer F.Cu) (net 25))
 (segment (start 118.237 98.425) (end 120.396 98.425) (width 0.25) (layer B.Cu) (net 25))
 (segment (start 120.396 98.425) (end 120.65 98.679) (width 0.25) (layer B.Cu) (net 25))
 (via (at 120.65 98.679) (size 0.6) (drill 0.4) (layers F.Cu B.Cu) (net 25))
 (segment (start 116.967 99.233) (end 116.967 99.096798) (width 0.25) (layer F.Cu) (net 25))
 (segment (start 116.967 99.096798) (end 117.638798 98.425) (width 0.25) (layer F.Cu) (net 25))
 (segment (start 117.638798 98.425) (end 118.237 98.425) (width 0.25) (layer F.Cu) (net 25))
 (via (at 118.237 98.425) (size 0.6) (drill 0.4) (layers F.Cu B.Cu) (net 25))
 (segment (start 116.1 100) (end 116.2 100) (width 0.25) (layer F.Cu) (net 25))
 (segment (start 116.2 100) (end 116.967 99.233) (width 0.25) (layer F.Cu) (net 25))
 (segment (start 115.6 93) (end 117.003 93) (width 0.25) (layer F.Cu) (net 26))
 (segment (start 118.2285 93.5905) (end 118.2285 94.75) (width 0.25) (layer F.Cu) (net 26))
 (segment (start 118.11 93.472) (end 118.2285 93.5905) (width 0.25) (layer F.Cu) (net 26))
 (segment (start 117.475 93.472) (end 118.11 93.472) (width 0.25) (layer F.Cu) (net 26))
 (segment (start 117.003 93) (end 117.475 93.472) (width 0.25) (layer F.Cu) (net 26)))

